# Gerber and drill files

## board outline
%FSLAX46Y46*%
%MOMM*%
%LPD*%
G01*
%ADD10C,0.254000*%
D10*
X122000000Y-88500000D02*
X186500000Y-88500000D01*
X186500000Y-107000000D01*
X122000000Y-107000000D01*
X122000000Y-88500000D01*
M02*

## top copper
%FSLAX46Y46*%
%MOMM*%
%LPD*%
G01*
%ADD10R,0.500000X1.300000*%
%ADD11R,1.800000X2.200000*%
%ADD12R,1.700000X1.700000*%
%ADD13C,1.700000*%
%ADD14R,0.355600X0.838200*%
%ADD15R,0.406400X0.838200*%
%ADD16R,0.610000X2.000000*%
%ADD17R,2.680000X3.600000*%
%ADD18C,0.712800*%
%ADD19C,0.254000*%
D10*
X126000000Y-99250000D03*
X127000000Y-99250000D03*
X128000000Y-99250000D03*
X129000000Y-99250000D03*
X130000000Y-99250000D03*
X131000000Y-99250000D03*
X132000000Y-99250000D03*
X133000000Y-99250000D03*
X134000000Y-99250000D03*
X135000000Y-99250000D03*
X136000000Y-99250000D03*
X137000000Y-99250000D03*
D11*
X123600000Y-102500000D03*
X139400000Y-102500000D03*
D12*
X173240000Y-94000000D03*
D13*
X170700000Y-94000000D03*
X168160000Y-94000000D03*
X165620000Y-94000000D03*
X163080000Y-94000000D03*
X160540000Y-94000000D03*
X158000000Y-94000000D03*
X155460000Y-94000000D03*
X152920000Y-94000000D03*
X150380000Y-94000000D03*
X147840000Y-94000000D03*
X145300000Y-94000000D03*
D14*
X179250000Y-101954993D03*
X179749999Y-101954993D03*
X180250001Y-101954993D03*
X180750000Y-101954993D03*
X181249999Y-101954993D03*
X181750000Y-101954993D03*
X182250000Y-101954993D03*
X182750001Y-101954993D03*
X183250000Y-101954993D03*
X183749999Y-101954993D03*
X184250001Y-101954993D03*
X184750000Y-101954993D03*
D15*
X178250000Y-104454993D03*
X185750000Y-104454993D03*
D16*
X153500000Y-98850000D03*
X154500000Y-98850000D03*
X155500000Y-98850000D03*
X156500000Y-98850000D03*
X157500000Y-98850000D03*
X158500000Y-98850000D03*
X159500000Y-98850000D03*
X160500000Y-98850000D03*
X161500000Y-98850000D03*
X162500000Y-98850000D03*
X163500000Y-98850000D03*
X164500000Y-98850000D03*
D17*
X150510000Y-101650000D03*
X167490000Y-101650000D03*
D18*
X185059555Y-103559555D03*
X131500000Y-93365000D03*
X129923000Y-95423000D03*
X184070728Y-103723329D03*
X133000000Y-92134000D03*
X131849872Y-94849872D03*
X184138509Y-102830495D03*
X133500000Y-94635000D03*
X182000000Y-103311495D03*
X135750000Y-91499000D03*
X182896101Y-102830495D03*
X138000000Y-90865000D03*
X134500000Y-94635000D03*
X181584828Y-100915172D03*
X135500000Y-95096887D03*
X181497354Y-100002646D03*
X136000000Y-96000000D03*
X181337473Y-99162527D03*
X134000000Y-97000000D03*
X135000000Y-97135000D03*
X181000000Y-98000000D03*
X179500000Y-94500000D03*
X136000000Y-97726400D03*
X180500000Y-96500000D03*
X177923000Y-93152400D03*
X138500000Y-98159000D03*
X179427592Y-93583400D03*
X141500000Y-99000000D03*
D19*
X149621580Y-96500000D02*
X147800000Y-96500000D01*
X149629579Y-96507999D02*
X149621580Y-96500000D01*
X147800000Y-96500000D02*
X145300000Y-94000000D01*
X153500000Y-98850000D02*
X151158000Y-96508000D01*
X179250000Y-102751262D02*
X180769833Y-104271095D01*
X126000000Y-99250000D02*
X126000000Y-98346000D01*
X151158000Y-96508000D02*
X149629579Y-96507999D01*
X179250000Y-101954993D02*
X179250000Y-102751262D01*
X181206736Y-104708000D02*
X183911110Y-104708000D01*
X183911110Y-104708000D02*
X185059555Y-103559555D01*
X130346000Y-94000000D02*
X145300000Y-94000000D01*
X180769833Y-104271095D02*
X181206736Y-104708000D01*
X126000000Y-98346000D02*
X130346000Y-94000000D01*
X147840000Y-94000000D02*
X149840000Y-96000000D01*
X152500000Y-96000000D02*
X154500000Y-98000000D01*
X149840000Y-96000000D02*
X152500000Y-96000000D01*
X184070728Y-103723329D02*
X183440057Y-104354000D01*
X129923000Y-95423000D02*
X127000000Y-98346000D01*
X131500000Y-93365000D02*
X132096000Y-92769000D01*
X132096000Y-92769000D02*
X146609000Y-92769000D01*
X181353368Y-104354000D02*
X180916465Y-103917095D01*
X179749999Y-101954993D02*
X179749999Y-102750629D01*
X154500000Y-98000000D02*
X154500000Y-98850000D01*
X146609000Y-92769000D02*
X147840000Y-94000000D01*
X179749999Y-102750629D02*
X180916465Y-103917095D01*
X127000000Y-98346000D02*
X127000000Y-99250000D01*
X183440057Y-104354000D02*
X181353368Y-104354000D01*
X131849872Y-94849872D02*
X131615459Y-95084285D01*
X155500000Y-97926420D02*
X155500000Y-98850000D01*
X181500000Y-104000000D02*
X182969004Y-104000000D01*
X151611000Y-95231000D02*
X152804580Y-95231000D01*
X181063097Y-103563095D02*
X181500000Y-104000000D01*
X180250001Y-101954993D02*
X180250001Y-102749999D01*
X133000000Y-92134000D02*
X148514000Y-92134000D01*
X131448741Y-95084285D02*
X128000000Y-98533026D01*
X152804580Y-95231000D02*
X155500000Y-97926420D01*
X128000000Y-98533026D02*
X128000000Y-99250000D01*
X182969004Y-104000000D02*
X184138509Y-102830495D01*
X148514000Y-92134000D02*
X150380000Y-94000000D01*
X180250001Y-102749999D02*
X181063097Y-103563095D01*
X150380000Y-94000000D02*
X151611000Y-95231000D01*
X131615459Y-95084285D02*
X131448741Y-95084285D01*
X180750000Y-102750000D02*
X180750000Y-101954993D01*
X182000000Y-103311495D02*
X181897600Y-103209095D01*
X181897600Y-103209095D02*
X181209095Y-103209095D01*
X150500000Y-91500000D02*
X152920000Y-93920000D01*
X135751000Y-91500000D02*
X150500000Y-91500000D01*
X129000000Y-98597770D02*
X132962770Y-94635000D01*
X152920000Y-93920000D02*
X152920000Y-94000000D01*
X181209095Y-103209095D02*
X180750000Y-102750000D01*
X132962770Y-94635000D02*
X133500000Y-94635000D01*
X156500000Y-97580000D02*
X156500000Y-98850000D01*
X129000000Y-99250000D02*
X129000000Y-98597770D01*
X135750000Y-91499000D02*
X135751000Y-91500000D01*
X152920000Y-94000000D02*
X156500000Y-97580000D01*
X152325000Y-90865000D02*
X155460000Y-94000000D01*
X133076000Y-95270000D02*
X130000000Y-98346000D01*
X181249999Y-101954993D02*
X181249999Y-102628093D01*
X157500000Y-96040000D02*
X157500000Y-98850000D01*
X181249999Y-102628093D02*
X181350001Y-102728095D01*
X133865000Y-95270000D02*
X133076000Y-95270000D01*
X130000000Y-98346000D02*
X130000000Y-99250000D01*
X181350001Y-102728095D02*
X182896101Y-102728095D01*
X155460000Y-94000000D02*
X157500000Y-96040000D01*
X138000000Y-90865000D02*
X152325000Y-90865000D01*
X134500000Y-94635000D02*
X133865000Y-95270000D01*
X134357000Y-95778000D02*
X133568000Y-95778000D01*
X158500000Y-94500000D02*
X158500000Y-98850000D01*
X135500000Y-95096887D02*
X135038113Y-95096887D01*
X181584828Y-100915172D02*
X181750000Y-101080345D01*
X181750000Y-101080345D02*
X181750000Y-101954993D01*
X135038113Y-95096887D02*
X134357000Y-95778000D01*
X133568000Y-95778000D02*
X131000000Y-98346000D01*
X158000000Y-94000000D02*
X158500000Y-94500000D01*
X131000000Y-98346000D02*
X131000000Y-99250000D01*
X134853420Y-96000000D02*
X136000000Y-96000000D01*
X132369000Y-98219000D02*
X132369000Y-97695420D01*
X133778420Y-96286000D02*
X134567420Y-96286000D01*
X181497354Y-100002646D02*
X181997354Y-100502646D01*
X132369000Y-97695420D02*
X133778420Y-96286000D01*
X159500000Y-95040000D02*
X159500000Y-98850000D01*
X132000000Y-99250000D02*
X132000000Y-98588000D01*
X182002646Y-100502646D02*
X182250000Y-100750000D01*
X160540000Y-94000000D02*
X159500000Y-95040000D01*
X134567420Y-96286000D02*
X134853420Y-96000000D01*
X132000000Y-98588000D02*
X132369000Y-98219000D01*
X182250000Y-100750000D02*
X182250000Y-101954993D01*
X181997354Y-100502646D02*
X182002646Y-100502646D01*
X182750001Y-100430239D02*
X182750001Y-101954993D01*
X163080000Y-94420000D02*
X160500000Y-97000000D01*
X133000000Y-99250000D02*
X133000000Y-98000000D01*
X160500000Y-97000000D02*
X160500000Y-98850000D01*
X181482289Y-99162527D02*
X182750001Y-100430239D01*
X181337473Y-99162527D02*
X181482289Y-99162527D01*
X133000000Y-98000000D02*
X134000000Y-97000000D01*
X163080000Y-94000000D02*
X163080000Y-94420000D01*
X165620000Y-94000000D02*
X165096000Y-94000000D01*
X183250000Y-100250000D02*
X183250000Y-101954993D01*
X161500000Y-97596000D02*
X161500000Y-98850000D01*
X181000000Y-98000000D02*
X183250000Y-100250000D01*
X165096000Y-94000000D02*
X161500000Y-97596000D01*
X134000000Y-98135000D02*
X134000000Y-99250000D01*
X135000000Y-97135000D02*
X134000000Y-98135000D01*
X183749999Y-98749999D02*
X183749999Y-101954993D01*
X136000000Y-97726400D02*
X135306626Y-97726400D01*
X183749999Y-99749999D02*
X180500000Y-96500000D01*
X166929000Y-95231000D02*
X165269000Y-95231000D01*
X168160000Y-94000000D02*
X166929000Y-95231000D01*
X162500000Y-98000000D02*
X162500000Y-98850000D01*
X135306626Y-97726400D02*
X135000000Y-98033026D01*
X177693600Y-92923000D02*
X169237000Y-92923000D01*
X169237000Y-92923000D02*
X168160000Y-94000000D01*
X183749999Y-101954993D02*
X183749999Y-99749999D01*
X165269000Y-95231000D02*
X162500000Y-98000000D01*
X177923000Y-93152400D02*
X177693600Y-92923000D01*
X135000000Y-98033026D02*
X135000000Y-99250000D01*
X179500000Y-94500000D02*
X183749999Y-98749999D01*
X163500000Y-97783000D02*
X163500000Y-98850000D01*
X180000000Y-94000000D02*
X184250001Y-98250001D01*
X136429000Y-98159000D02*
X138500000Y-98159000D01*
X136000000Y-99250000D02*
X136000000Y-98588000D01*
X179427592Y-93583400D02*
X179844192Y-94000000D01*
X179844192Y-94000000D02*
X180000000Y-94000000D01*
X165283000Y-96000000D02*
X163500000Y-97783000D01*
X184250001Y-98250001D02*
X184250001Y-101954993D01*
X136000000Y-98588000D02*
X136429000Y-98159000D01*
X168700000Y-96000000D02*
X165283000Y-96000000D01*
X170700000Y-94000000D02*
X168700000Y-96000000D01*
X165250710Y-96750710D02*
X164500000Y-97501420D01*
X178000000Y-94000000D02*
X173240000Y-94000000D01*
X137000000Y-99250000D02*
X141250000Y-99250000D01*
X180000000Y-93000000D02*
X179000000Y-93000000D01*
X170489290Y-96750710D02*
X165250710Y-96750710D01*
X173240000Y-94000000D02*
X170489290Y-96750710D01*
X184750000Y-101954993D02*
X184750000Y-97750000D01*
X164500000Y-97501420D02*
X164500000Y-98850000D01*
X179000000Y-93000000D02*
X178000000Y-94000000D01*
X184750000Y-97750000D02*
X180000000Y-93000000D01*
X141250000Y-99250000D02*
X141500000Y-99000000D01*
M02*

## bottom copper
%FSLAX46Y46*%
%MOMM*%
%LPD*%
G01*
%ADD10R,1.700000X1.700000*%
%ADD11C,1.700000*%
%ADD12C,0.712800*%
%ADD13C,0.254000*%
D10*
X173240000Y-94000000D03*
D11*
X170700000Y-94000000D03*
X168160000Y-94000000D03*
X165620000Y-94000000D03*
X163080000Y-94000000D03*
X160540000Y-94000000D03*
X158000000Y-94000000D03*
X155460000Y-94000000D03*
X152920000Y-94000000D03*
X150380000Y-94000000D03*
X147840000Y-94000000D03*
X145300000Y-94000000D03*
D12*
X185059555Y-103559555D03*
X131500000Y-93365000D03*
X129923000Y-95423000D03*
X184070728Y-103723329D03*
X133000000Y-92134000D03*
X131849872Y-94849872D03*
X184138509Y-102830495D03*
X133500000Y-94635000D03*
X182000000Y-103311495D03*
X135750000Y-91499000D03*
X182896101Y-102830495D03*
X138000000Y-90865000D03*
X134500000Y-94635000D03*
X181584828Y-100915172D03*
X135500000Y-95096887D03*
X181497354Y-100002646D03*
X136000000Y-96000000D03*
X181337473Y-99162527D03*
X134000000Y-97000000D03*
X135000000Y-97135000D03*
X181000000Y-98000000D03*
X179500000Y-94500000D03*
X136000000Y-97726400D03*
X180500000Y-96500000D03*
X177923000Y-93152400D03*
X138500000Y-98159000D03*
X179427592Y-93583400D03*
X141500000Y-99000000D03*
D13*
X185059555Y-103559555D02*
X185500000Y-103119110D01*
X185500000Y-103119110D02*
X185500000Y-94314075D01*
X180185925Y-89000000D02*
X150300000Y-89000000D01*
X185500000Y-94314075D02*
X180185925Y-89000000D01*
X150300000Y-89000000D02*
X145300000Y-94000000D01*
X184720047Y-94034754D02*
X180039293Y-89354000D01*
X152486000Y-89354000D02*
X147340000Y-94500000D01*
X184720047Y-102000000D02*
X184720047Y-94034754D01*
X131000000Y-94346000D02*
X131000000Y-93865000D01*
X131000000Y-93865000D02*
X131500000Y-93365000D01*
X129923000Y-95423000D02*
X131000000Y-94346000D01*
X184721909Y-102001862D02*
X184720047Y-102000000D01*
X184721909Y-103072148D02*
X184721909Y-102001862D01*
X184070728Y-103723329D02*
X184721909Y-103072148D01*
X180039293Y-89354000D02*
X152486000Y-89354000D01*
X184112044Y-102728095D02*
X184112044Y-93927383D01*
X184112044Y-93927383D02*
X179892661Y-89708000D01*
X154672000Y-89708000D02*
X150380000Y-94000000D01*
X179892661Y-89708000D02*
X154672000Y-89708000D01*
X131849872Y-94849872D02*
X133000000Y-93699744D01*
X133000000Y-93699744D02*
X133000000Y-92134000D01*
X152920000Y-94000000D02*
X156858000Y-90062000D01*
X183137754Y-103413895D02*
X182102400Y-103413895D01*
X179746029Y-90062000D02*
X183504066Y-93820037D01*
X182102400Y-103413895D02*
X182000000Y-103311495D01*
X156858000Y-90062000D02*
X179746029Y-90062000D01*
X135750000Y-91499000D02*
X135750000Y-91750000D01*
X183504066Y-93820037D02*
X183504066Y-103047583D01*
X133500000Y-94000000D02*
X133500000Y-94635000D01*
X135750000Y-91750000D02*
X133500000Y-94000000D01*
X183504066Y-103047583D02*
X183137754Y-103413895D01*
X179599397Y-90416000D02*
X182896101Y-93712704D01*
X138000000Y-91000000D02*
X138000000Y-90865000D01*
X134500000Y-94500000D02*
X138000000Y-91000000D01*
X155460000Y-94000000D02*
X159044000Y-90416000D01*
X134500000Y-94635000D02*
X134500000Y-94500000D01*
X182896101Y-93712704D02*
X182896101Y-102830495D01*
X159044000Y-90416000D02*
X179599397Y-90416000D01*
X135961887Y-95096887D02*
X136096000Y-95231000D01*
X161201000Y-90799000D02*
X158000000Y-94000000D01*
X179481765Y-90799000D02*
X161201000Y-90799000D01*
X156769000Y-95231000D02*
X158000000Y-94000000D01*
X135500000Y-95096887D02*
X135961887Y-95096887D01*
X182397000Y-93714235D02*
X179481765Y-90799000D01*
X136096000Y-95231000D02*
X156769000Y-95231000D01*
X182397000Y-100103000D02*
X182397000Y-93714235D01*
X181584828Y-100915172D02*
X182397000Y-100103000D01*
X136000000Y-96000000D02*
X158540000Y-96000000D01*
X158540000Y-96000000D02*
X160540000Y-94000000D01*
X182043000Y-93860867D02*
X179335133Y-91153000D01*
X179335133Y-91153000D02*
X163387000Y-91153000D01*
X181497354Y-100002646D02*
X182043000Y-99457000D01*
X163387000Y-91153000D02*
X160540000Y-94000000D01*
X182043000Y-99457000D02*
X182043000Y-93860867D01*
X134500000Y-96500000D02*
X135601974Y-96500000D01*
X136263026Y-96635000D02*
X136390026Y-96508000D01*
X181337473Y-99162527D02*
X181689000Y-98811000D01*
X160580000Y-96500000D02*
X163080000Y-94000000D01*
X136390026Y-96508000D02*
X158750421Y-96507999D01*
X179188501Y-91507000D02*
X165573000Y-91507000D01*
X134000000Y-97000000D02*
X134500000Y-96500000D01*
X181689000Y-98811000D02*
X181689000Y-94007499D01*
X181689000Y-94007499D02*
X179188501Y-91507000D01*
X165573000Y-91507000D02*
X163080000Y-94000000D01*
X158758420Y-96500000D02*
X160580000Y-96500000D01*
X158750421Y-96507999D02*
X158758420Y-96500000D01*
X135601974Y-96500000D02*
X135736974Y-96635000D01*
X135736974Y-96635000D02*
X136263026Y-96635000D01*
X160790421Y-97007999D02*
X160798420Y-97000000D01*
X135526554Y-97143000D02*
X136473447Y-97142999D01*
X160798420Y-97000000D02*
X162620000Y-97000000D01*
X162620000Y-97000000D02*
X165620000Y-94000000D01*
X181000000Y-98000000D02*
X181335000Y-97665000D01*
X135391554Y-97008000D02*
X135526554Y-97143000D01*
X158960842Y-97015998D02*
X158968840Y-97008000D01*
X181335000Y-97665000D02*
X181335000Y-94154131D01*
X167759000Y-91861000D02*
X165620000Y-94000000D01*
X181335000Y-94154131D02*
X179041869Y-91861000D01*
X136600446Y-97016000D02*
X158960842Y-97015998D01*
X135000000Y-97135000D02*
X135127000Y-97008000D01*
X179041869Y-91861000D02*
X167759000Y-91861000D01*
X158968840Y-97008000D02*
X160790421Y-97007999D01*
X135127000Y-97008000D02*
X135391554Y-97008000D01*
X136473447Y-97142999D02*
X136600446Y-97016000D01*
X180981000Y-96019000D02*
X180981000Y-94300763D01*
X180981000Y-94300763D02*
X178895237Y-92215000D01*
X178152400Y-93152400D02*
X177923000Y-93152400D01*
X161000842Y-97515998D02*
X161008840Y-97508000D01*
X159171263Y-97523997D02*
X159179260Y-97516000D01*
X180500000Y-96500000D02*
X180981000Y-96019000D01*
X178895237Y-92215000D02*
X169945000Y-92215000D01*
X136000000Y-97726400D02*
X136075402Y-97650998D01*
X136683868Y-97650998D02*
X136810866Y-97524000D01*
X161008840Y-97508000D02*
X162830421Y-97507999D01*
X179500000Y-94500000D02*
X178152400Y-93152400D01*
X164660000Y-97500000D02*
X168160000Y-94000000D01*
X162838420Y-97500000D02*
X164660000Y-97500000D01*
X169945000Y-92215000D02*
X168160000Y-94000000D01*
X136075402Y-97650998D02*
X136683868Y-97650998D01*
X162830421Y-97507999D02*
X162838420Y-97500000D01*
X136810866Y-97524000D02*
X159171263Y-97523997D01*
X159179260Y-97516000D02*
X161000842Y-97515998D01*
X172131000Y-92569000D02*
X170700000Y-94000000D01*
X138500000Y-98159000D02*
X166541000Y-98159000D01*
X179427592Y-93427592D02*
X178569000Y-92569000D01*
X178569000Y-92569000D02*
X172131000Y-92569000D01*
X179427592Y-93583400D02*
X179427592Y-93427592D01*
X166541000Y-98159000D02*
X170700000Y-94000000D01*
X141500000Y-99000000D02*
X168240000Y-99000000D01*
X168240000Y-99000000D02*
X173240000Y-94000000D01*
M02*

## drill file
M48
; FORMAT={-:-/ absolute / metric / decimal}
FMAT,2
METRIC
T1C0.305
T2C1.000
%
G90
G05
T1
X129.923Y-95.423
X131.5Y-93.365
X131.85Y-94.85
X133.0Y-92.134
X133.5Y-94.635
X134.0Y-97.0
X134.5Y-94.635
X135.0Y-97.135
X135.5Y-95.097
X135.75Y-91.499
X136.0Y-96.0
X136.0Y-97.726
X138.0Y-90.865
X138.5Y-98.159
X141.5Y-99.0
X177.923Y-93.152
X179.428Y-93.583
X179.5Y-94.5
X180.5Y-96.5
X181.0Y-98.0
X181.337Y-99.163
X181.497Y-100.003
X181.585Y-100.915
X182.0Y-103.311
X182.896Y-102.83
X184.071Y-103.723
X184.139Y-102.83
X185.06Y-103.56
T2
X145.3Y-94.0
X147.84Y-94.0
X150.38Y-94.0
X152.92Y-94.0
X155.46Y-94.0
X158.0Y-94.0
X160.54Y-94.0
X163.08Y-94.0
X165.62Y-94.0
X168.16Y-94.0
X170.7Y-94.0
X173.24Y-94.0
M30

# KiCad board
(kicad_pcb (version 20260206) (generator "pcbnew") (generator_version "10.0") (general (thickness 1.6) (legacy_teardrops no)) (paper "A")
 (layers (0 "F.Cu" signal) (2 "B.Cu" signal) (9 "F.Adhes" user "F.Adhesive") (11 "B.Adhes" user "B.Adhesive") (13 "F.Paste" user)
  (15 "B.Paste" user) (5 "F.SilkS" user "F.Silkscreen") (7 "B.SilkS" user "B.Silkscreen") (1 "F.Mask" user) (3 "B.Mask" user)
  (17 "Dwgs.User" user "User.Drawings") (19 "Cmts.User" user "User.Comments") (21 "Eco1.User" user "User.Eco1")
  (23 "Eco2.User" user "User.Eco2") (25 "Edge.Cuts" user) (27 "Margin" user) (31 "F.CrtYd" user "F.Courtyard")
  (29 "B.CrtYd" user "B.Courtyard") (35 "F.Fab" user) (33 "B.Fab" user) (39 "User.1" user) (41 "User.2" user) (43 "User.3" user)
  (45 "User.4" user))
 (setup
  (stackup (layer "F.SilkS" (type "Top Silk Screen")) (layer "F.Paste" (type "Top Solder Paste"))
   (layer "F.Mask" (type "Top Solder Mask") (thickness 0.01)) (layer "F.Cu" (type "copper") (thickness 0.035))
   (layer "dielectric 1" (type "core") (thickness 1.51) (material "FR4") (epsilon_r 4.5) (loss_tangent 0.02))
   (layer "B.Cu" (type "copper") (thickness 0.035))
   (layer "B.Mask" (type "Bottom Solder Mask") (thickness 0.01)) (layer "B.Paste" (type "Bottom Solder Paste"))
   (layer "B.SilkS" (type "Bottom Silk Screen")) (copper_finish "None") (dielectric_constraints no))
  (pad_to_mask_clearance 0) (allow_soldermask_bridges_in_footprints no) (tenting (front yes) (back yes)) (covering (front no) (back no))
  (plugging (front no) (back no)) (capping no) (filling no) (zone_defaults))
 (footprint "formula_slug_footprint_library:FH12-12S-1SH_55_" (layer "F.Cu") (at 131.5 100.05)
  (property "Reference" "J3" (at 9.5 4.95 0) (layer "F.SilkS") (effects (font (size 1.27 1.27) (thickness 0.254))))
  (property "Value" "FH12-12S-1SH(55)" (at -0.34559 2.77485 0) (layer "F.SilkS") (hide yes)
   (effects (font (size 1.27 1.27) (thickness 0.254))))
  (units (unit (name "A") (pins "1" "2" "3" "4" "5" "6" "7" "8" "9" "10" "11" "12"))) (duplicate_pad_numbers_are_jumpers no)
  (pad "1" smd rect (at -5.5 -0.8) (size 0.5 1.3) (layers "F.Cu" "F.Mask" "F.Paste") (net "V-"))
  (pad "2" smd rect (at -4.5 -0.8) (size 0.5 1.3) (layers "F.Cu" "F.Mask" "F.Paste") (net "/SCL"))
  (pad "3" smd rect (at -3.5 -0.8) (size 0.5 1.3) (layers "F.Cu" "F.Mask" "F.Paste") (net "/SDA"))
  (pad "4" smd rect (at -2.5 -0.8) (size 0.5 1.3) (layers "F.Cu" "F.Mask" "F.Paste") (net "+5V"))
  (pad "5" smd rect (at -1.5 -0.8) (size 0.5 1.3) (layers "F.Cu" "F.Mask" "F.Paste") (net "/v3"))
  (pad "6" smd rect (at -0.5 -0.8) (size 0.5 1.3) (layers "F.Cu" "F.Mask" "F.Paste") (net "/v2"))
  (pad "7" smd rect (at 0.5 -0.8) (size 0.5 1.3) (layers "F.Cu" "F.Mask" "F.Paste") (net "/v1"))
  (pad "8" smd rect (at 1.5 -0.8) (size 0.5 1.3) (layers "F.Cu" "F.Mask" "F.Paste") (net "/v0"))
  (pad "9" smd rect (at 2.5 -0.8) (size 0.5 1.3) (layers "F.Cu" "F.Mask" "F.Paste") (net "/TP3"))
  (pad "10" smd rect (at 3.5 -0.8) (size 0.5 1.3) (layers "F.Cu" "F.Mask" "F.Paste") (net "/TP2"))
  (pad "11" smd rect (at 4.5 -0.8) (size 0.5 1.3) (layers "F.Cu" "F.Mask" "F.Paste") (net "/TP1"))
  (pad "12" smd rect (at 5.5 -0.8) (size 0.5 1.3) (layers "F.Cu" "F.Mask" "F.Paste") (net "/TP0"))
  (pad "13" smd rect (at -7.9 2.45) (size 1.8 2.2) (layers "F.Cu" "F.Mask" "F.Paste"))
  (pad "14" smd rect (at 7.9 2.45) (size 1.8 2.2) (layers "F.Cu" "F.Mask" "F.Paste")))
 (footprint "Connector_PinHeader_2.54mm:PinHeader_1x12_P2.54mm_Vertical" (layer "F.Cu") (at 173.24 94 -90)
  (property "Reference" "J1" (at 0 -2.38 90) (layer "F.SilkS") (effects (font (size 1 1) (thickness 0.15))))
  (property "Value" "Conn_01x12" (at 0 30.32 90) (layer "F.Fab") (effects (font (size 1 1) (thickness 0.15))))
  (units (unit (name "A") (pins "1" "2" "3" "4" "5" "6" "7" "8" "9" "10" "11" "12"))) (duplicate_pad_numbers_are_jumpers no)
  (pad "1" thru_hole rect (at 0 0 270) (size 1.7 1.7) (drill 1) (layers "*.Cu" "*.Mask") (remove_unused_layers no) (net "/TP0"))
  (pad "2" thru_hole circle (at 0 2.54 270) (size 1.7 1.7) (drill 1) (layers "*.Cu" "*.Mask") (remove_unused_layers no) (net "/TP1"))
  (pad "3" thru_hole circle (at 0 5.08 270) (size 1.7 1.7) (drill 1) (layers "*.Cu" "*.Mask") (remove_unused_layers no) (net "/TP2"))
  (pad "4" thru_hole circle (at 0 7.62 270) (size 1.7 1.7) (drill 1) (layers "*.Cu" "*.Mask") (remove_unused_layers no) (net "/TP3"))
  (pad "5" thru_hole circle (at 0 10.16 270) (size 1.7 1.7) (drill 1) (layers "*.Cu" "*.Mask") (remove_unused_layers no) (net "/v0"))
  (pad "6" thru_hole circle (at 0 12.7 270) (size 1.7 1.7) (drill 1) (layers "*.Cu" "*.Mask") (remove_unused_layers no) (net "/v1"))
  (pad "7" thru_hole circle (at 0 15.24 270) (size 1.7 1.7) (drill 1) (layers "*.Cu" "*.Mask") (remove_unused_layers no) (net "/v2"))
  (pad "8" thru_hole circle (at 0 17.78 270) (size 1.7 1.7) (drill 1) (layers "*.Cu" "*.Mask") (remove_unused_layers no) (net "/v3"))
  (pad "9" thru_hole circle (at 0 20.32 270) (size 1.7 1.7) (drill 1) (layers "*.Cu" "*.Mask") (remove_unused_layers no) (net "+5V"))
  (pad "10" thru_hole circle (at 0 22.86 270) (size 1.7 1.7) (drill 1) (layers "*.Cu" "*.Mask") (remove_unused_layers no) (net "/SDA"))
  (pad "11" thru_hole circle (at 0 25.4 270) (size 1.7 1.7) (drill 1) (layers "*.Cu" "*.Mask") (remove_unused_layers no) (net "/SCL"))
  (pad "12" thru_hole circle (at 0 27.94 270) (size 1.7 1.7) (drill 1) (layers "*.Cu" "*.Mask") (remove_unused_layers no) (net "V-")))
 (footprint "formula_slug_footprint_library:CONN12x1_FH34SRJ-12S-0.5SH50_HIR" (layer "F.Cu") (at 182 103)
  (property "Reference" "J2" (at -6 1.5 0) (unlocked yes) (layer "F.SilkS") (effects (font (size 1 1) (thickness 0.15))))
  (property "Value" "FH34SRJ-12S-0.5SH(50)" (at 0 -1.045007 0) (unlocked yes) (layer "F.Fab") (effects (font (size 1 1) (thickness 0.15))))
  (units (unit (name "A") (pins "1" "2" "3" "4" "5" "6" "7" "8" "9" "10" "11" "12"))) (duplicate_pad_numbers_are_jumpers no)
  (pad "1" smd rect (at -2.75 -1.045007) (size 0.3556 0.8382) (layers "F.Cu" "F.Mask" "F.Paste") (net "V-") (clearance 0.1))
  (pad "2" smd rect (at -2.250001 -1.045007) (size 0.3556 0.8382) (layers "F.Cu" "F.Mask" "F.Paste") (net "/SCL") (clearance 0.1))
  (pad "3" smd rect (at -1.749999 -1.045007) (size 0.3556 0.8382) (layers "F.Cu" "F.Mask" "F.Paste") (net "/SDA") (clearance 0.1))
  (pad "4" smd rect (at -1.25 -1.045007) (size 0.3556 0.8382) (layers "F.Cu" "F.Mask" "F.Paste") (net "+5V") (clearance 0.1))
  (pad "5" smd rect (at -0.750001 -1.045007) (size 0.3556 0.8382) (layers "F.Cu" "F.Mask" "F.Paste") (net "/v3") (clearance 0.1))
  (pad "6" smd rect (at -0.25 -1.045007) (size 0.3556 0.8382) (layers "F.Cu" "F.Mask" "F.Paste") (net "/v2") (clearance 0.1))
  (pad "7" smd rect (at 0.25 -1.045007) (size 0.3556 0.8382) (layers "F.Cu" "F.Mask" "F.Paste") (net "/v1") (clearance 0.1))
  (pad "8" smd rect (at 0.750001 -1.045007) (size 0.3556 0.8382) (layers "F.Cu" "F.Mask" "F.Paste") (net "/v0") (clearance 0.1))
  (pad "9" smd rect (at 1.25 -1.045007) (size 0.3556 0.8382) (layers "F.Cu" "F.Mask" "F.Paste") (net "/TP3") (clearance 0.1))
  (pad "10" smd rect (at 1.749999 -1.045007) (size 0.3556 0.8382) (layers "F.Cu" "F.Mask" "F.Paste") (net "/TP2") (clearance 0.1))
  (pad "11" smd rect (at 2.250001 -1.045007) (size 0.3556 0.8382) (layers "F.Cu" "F.Mask" "F.Paste") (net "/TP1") (clearance 0.1))
  (pad "12" smd rect (at 2.75 -1.045007) (size 0.3556 0.8382) (layers "F.Cu" "F.Mask" "F.Paste") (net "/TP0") (clearance 0.1))
  (pad "13" smd rect (at -3.75 1.454993) (size 0.4064 0.8382) (layers "F.Cu" "F.Mask" "F.Paste"))
  (pad "14" smd rect (at 3.75 1.454993) (size 0.4064 0.8382) (layers "F.Cu" "F.Mask" "F.Paste")))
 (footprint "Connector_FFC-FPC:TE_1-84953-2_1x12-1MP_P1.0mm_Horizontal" (layer "F.Cu") (at 159 100.65)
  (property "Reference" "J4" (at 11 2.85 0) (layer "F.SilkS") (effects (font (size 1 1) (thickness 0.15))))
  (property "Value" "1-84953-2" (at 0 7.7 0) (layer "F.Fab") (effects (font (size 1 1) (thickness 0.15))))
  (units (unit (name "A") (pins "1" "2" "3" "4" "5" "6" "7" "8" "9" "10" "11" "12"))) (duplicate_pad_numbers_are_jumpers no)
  (pad "1" smd rect (at -5.5 -1.8) (size 0.61 2) (layers "F.Cu" "F.Mask" "F.Paste") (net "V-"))
  (pad "2" smd rect (at -4.5 -1.8) (size 0.61 2) (layers "F.Cu" "F.Mask" "F.Paste") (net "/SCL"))
  (pad "3" smd rect (at -3.5 -1.8) (size 0.61 2) (layers "F.Cu" "F.Mask" "F.Paste") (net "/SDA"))
  (pad "4" smd rect (at -2.5 -1.8) (size 0.61 2) (layers "F.Cu" "F.Mask" "F.Paste") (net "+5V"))
  (pad "5" smd rect (at -1.5 -1.8) (size 0.61 2) (layers "F.Cu" "F.Mask" "F.Paste") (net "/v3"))
  (pad "6" smd rect (at -0.5 -1.8) (size 0.61 2) (layers "F.Cu" "F.Mask" "F.Paste") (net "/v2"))
  (pad "7" smd rect (at 0.5 -1.8) (size 0.61 2) (layers "F.Cu" "F.Mask" "F.Paste") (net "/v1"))
  (pad "8" smd rect (at 1.5 -1.8) (size 0.61 2) (layers "F.Cu" "F.Mask" "F.Paste") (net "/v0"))
  (pad "9" smd rect (at 2.5 -1.8) (size 0.61 2) (layers "F.Cu" "F.Mask" "F.Paste") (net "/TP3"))
  (pad "10" smd rect (at 3.5 -1.8) (size 0.61 2) (layers "F.Cu" "F.Mask" "F.Paste") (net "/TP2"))
  (pad "11" smd rect (at 4.5 -1.8) (size 0.61 2) (layers "F.Cu" "F.Mask" "F.Paste") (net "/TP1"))
  (pad "12" smd rect (at 5.5 -1.8) (size 0.61 2) (layers "F.Cu" "F.Mask" "F.Paste") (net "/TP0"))
  (pad "MP" smd rect (at -8.49 1) (size 2.68 3.6) (layers "F.Cu" "F.Mask" "F.Paste"))
  (pad "MP" smd rect (at 8.49 1) (size 2.68 3.6) (layers "F.Cu" "F.Mask" "F.Paste")))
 (gr_rect (start 122 88.5) (end 186.5 107) (stroke (width 0.254) (type solid)) (fill no) (layer "Edge.Cuts"))
 (segment (start 149.62158 96.5) (end 147.8 96.5) (width 0.254) (layer "F.Cu") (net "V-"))
 (segment (start 149.629579 96.507999) (end 149.62158 96.5) (width 0.254) (layer "F.Cu") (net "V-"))
 (segment (start 147.8 96.5) (end 145.3 94) (width 0.254) (layer "F.Cu") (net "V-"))
 (segment (start 153.5 98.85) (end 151.158 96.508) (width 0.254) (layer "F.Cu") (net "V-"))
 (segment (start 179.25 102.751262) (end 180.769833 104.271095) (width 0.254) (layer "F.Cu") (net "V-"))
 (segment (start 126 99.25) (end 126 98.346) (width 0.254) (layer "F.Cu") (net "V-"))
 (segment (start 151.158 96.508) (end 149.629579 96.507999) (width 0.254) (layer "F.Cu") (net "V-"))
 (segment (start 179.25 101.954993) (end 179.25 102.751262) (width 0.254) (layer "F.Cu") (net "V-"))
 (segment (start 181.206736 104.708) (end 183.91111 104.708) (width 0.254) (layer "F.Cu") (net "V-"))
 (segment (start 183.91111 104.708) (end 185.059555 103.559555) (width 0.254) (layer "F.Cu") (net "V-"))
 (segment (start 130.346 94) (end 145.3 94) (width 0.254) (layer "F.Cu") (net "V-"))
 (segment (start 180.769833 104.271095) (end 181.206736 104.708) (width 0.254) (layer "F.Cu") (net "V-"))
 (segment (start 126 98.346) (end 130.346 94) (width 0.254) (layer "F.Cu") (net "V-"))
 (via (at 185.059555 103.559555) (size 0.7128) (drill 0.3048) (layers "F.Cu" "B.Cu") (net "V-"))
 (segment (start 185.059555 103.559555) (end 185.5 103.11911) (width 0.254) (layer "B.Cu") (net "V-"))
 (segment (start 185.5 103.11911) (end 185.5 94.314075) (width 0.254) (layer "B.Cu") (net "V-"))
 (segment (start 180.185925 89) (end 150.3 89) (width 0.254) (layer "B.Cu") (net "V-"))
 (segment (start 185.5 94.314075) (end 180.185925 89) (width 0.254) (layer "B.Cu") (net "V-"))
 (segment (start 150.3 89) (end 145.3 94) (width 0.254) (layer "B.Cu") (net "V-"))
 (segment (start 147.84 94) (end 149.84 96) (width 0.254) (layer "F.Cu") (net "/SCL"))
 (segment (start 152.5 96) (end 154.5 98) (width 0.254) (layer "F.Cu") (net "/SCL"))
 (segment (start 149.84 96) (end 152.5 96) (width 0.254) (layer "F.Cu") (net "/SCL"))
 (segment (start 184.070728 103.723329) (end 183.440057 104.354) (width 0.254) (layer "F.Cu") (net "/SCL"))
 (segment (start 129.923 95.423) (end 127 98.346) (width 0.254) (layer "F.Cu") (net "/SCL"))
 (segment (start 131.5 93.365) (end 132.096 92.769) (width 0.254) (layer "F.Cu") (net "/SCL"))
 (segment (start 132.096 92.769) (end 146.609 92.769) (width 0.254) (layer "F.Cu") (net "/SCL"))
 (segment (start 181.353368 104.354) (end 180.916465 103.917095) (width 0.254) (layer "F.Cu") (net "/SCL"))
 (segment (start 179.749999 101.954993) (end 179.749999 102.750629) (width 0.254) (layer "F.Cu") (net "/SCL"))
 (segment (start 154.5 98) (end 154.5 98.85) (width 0.254) (layer "F.Cu") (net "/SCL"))
 (segment (start 146.609 92.769) (end 147.84 94) (width 0.254) (layer "F.Cu") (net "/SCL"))
 (segment (start 179.749999 102.750629) (end 180.916465 103.917095) (width 0.254) (layer "F.Cu") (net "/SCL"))
 (segment (start 127 98.346) (end 127 99.25) (width 0.254) (layer "F.Cu") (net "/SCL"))
 (segment (start 183.440057 104.354) (end 181.353368 104.354) (width 0.254) (layer "F.Cu") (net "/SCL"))
 (via (at 131.5 93.365) (size 0.7128) (drill 0.3048) (layers "F.Cu" "B.Cu") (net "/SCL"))
 (via (at 129.923 95.423) (size 0.7128) (drill 0.3048) (layers "F.Cu" "B.Cu") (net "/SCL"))
 (via (at 184.070728 103.723329) (size 0.7128) (drill 0.3048) (layers "F.Cu" "B.Cu") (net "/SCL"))
 (segment (start 184.720047 94.034754) (end 180.039293 89.354) (width 0.254) (layer "B.Cu") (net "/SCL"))
 (segment (start 152.486 89.354) (end 147.34 94.5) (width 0.254) (layer "B.Cu") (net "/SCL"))
 (segment (start 184.720047 102) (end 184.720047 94.034754) (width 0.254) (layer "B.Cu") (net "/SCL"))
 (segment (start 131 94.346) (end 131 93.865) (width 0.254) (layer "B.Cu") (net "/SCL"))
 (segment (start 131 93.865) (end 131.5 93.365) (width 0.254) (layer "B.Cu") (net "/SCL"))
 (segment (start 129.923 95.423) (end 131 94.346) (width 0.254) (layer "B.Cu") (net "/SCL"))
 (segment (start 184.721909 102.001862) (end 184.720047 102) (width 0.254) (layer "B.Cu") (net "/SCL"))
 (segment (start 184.721909 103.072148) (end 184.721909 102.001862) (width 0.254) (layer "B.Cu") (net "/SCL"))
 (segment (start 184.070728 103.723329) (end 184.721909 103.072148) (width 0.254) (layer "B.Cu") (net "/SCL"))
 (segment (start 180.039293 89.354) (end 152.486 89.354) (width 0.254) (layer "B.Cu") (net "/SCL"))
 (segment (start 131.849872 94.849872) (end 131.615459 95.084285) (width 0.254) (layer "F.Cu") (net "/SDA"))
 (segment (start 155.5 97.92642) (end 155.5 98.85) (width 0.254) (layer "F.Cu") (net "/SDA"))
 (segment (start 181.5 104) (end 182.969004 104) (width 0.254) (layer "F.Cu") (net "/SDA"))
 (segment (start 151.611 95.231) (end 152.80458 95.231) (width 0.254) (layer "F.Cu") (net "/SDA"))
 (segment (start 181.063097 103.563095) (end 181.5 104) (width 0.254) (layer "F.Cu") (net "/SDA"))
 (segment (start 180.250001 101.954993) (end 180.250001 102.749999) (width 0.254) (layer "F.Cu") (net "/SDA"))
 (segment (start 133 92.134) (end 148.514 92.134) (width 0.254) (layer "F.Cu") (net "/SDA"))
 (segment (start 131.448741 95.084285) (end 128 98.533026) (width 0.254) (layer "F.Cu") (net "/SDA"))
 (segment (start 152.80458 95.231) (end 155.5 97.92642) (width 0.254) (layer "F.Cu") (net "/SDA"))
 (segment (start 128 98.533026) (end 128 99.25) (width 0.254) (layer "F.Cu") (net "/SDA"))
 (segment (start 182.969004 104) (end 184.138509 102.830495) (width 0.254) (layer "F.Cu") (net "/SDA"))
 (segment (start 148.514 92.134) (end 150.38 94) (width 0.254) (layer "F.Cu") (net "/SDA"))
 (segment (start 180.250001 102.749999) (end 181.063097 103.563095) (width 0.254) (layer "F.Cu") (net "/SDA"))
 (segment (start 150.38 94) (end 151.611 95.231) (width 0.254) (layer "F.Cu") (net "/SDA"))
 (segment (start 131.615459 95.084285) (end 131.448741 95.084285) (width 0.254) (layer "F.Cu") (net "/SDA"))
 (via (at 133 92.134) (size 0.7128) (drill 0.3048) (layers "F.Cu" "B.Cu") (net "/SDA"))
 (via (at 131.849872 94.849872) (size 0.7128) (drill 0.3048) (layers "F.Cu" "B.Cu") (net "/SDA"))
 (via (at 184.138509 102.830495) (size 0.7128) (drill 0.3048) (layers "F.Cu" "B.Cu") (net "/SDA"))
 (segment (start 184.112044 102.728095) (end 184.112044 93.927383) (width 0.254) (layer "B.Cu") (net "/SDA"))
 (segment (start 184.112044 93.927383) (end 179.892661 89.708) (width 0.254) (layer "B.Cu") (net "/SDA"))
 (segment (start 154.672 89.708) (end 150.38 94) (width 0.254) (layer "B.Cu") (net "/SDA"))
 (segment (start 179.892661 89.708) (end 154.672 89.708) (width 0.254) (layer "B.Cu") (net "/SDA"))
 (segment (start 131.849872 94.849872) (end 133 93.699744) (width 0.254) (layer "B.Cu") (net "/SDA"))
 (segment (start 133 93.699744) (end 133 92.134) (width 0.254) (layer "B.Cu") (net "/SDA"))
 (segment (start 180.75 102.75) (end 180.75 101.954993) (width 0.254) (layer "F.Cu") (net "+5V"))
 (segment (start 182 103.311495) (end 181.8976 103.209095) (width 0.254) (layer "F.Cu") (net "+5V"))
 (segment (start 181.8976 103.209095) (end 181.209095 103.209095) (width 0.254) (layer "F.Cu") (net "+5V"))
 (segment (start 150.5 91.5) (end 152.92 93.92) (width 0.254) (layer "F.Cu") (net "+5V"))
 (segment (start 135.751 91.5) (end 150.5 91.5) (width 0.254) (layer "F.Cu") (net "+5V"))
 (segment (start 129 98.59777) (end 132.96277 94.635) (width 0.254) (layer "F.Cu") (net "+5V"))
 (segment (start 152.92 93.92) (end 152.92 94) (width 0.254) (layer "F.Cu") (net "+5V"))
 (segment (start 181.209095 103.209095) (end 180.75 102.75) (width 0.254) (layer "F.Cu") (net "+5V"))
 (segment (start 132.96277 94.635) (end 133.5 94.635) (width 0.254) (layer "F.Cu") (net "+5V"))
 (segment (start 156.5 97.58) (end 156.5 98.85) (width 0.254) (layer "F.Cu") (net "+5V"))
 (segment (start 129 99.25) (end 129 98.59777) (width 0.254) (layer "F.Cu") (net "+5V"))
 (segment (start 135.75 91.499) (end 135.751 91.5) (width 0.254) (layer "F.Cu") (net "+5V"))
 (segment (start 152.92 94) (end 156.5 97.58) (width 0.254) (layer "F.Cu") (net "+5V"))
 (via (at 133.5 94.635) (size 0.7128) (drill 0.3048) (layers "F.Cu" "B.Cu") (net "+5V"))
 (via (at 182 103.311495) (size 0.7128) (drill 0.3048) (layers "F.Cu" "B.Cu") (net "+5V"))
 (via (at 135.75 91.499) (size 0.7128) (drill 0.3048) (layers "F.Cu" "B.Cu") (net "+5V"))
 (segment (start 152.92 94) (end 156.858 90.062) (width 0.254) (layer "B.Cu") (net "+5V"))
 (segment (start 183.137754 103.413895) (end 182.1024 103.413895) (width 0.254) (layer "B.Cu") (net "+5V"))
 (segment (start 179.746029 90.062) (end 183.504066 93.820037) (width 0.254) (layer "B.Cu") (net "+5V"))
 (segment (start 182.1024 103.413895) (end 182 103.311495) (width 0.254) (layer "B.Cu") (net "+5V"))
 (segment (start 156.858 90.062) (end 179.746029 90.062) (width 0.254) (layer "B.Cu") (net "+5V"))
 (segment (start 135.75 91.499) (end 135.75 91.75) (width 0.254) (layer "B.Cu") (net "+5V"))
 (segment (start 183.504066 93.820037) (end 183.504066 103.047583) (width 0.254) (layer "B.Cu") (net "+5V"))
 (segment (start 133.5 94) (end 133.5 94.635) (width 0.254) (layer "B.Cu") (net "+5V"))
 (segment (start 135.75 91.75) (end 133.5 94) (width 0.254) (layer "B.Cu") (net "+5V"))
 (segment (start 183.504066 103.047583) (end 183.137754 103.413895) (width 0.254) (layer "B.Cu") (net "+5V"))
 (segment (start 152.325 90.865) (end 155.46 94) (width 0.254) (layer "F.Cu") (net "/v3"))
 (segment (start 133.076 95.27) (end 130 98.346) (width 0.254) (layer "F.Cu") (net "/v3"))
 (segment (start 181.249999 101.954993) (end 181.249999 102.628093) (width 0.254) (layer "F.Cu") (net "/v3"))
 (segment (start 157.5 96.04) (end 157.5 98.85) (width 0.254) (layer "F.Cu") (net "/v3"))
 (segment (start 181.249999 102.628093) (end 181.350001 102.728095) (width 0.254) (layer "F.Cu") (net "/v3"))
 (segment (start 133.865 95.27) (end 133.076 95.27) (width 0.254) (layer "F.Cu") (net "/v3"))
 (segment (start 130 98.346) (end 130 99.25) (width 0.254) (layer "F.Cu") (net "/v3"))
 (segment (start 181.350001 102.728095) (end 182.896101 102.728095) (width 0.254) (layer "F.Cu") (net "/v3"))
 (segment (start 155.46 94) (end 157.5 96.04) (width 0.254) (layer "F.Cu") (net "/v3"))
 (segment (start 138 90.865) (end 152.325 90.865) (width 0.254) (layer "F.Cu") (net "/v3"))
 (segment (start 134.5 94.635) (end 133.865 95.27) (width 0.254) (layer "F.Cu") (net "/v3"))
 (via (at 182.896101 102.830495) (size 0.7128) (drill 0.3048) (layers "F.Cu" "B.Cu") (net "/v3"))
 (via (at 138 90.865) (size 0.7128) (drill 0.3048) (layers "F.Cu" "B.Cu") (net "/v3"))
 (via (at 134.5 94.635) (size 0.7128) (drill 0.3048) (layers "F.Cu" "B.Cu") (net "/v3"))
 (segment (start 179.599397 90.416) (end 182.896101 93.712704) (width 0.254) (layer "B.Cu") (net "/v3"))
 (segment (start 138 91) (end 138 90.865) (width 0.254) (layer "B.Cu") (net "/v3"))
 (segment (start 134.5 94.5) (end 138 91) (width 0.254) (layer "B.Cu") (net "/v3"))
 (segment (start 155.46 94) (end 159.044 90.416) (width 0.254) (layer "B.Cu") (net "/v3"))
 (segment (start 134.5 94.635) (end 134.5 94.5) (width 0.254) (layer "B.Cu") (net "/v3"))
 (segment (start 182.896101 93.712704) (end 182.896101 102.830495) (width 0.254) (layer "B.Cu") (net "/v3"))
 (segment (start 159.044 90.416) (end 179.599397 90.416) (width 0.254) (layer "B.Cu") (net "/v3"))
 (segment (start 134.357 95.778) (end 133.568 95.778) (width 0.254) (layer "F.Cu") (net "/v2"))
 (segment (start 158.5 94.5) (end 158.5 98.85) (width 0.254) (layer "F.Cu") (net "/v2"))
 (segment (start 135.5 95.096887) (end 135.038113 95.096887) (width 0.254) (layer "F.Cu") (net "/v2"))
 (segment (start 181.584828 100.915172) (end 181.75 101.080345) (width 0.254) (layer "F.Cu") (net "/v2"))
 (segment (start 181.75 101.080345) (end 181.75 101.954993) (width 0.254) (layer "F.Cu") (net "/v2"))
 (segment (start 135.038113 95.096887) (end 134.357 95.778) (width 0.254) (layer "F.Cu") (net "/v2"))
 (segment (start 133.568 95.778) (end 131 98.346) (width 0.254) (layer "F.Cu") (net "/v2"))
 (segment (start 158 94) (end 158.5 94.5) (width 0.254) (layer "F.Cu") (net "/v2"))
 (segment (start 131 98.346) (end 131 99.25) (width 0.254) (layer "F.Cu") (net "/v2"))
 (via (at 181.584828 100.915172) (size 0.7128) (drill 0.3048) (layers "F.Cu" "B.Cu") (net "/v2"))
 (via (at 135.5 95.096887) (size 0.7128) (drill 0.3048) (layers "F.Cu" "B.Cu") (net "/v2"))
 (segment (start 135.961887 95.096887) (end 136.096 95.231) (width 0.254) (layer "B.Cu") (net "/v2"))
 (segment (start 161.201 90.799) (end 158 94) (width 0.254) (layer "B.Cu") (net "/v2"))
 (segment (start 179.481765 90.799) (end 161.201 90.799) (width 0.254) (layer "B.Cu") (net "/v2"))
 (segment (start 156.769 95.231) (end 158 94) (width 0.254) (layer "B.Cu") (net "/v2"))
 (segment (start 135.5 95.096887) (end 135.961887 95.096887) (width 0.254) (layer "B.Cu") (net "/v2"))
 (segment (start 182.397 93.714235) (end 179.481765 90.799) (width 0.254) (layer "B.Cu") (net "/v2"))
 (segment (start 136.096 95.231) (end 156.769 95.231) (width 0.254) (layer "B.Cu") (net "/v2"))
 (segment (start 182.397 100.103) (end 182.397 93.714235) (width 0.254) (layer "B.Cu") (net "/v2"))
 (segment (start 181.584828 100.915172) (end 182.397 100.103) (width 0.254) (layer "B.Cu") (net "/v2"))
 (segment (start 134.85342 96) (end 136 96) (width 0.254) (layer "F.Cu") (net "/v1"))
 (segment (start 132.369 98.219) (end 132.369 97.69542) (width 0.254) (layer "F.Cu") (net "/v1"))
 (segment (start 133.77842 96.286) (end 134.56742 96.286) (width 0.254) (layer "F.Cu") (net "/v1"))
 (segment (start 181.497354 100.002646) (end 181.997354 100.502646) (width 0.254) (layer "F.Cu") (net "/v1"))
 (segment (start 132.369 97.69542) (end 133.77842 96.286) (width 0.254) (layer "F.Cu") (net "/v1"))
 (segment (start 159.5 95.04) (end 159.5 98.85) (width 0.254) (layer "F.Cu") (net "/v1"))
 (segment (start 132 99.25) (end 132 98.588) (width 0.254) (layer "F.Cu") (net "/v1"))
 (segment (start 182.002646 100.502646) (end 182.25 100.75) (width 0.254) (layer "F.Cu") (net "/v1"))
 (segment (start 160.54 94) (end 159.5 95.04) (width 0.254) (layer "F.Cu") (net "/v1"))
 (segment (start 134.56742 96.286) (end 134.85342 96) (width 0.254) (layer "F.Cu") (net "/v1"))
 (segment (start 132 98.588) (end 132.369 98.219) (width 0.254) (layer "F.Cu") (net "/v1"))
 (segment (start 182.25 100.75) (end 182.25 101.954993) (width 0.254) (layer "F.Cu") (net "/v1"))
 (segment (start 181.997354 100.502646) (end 182.002646 100.502646) (width 0.254) (layer "F.Cu") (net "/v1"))
 (via (at 181.497354 100.002646) (size 0.7128) (drill 0.3048) (layers "F.Cu" "B.Cu") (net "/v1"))
 (via (at 136 96) (size 0.7128) (drill 0.3048) (layers "F.Cu" "B.Cu") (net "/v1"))
 (segment (start 136 96) (end 158.54 96) (width 0.254) (layer "B.Cu") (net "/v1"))
 (segment (start 158.54 96) (end 160.54 94) (width 0.254) (layer "B.Cu") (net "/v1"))
 (segment (start 182.043 93.860867) (end 179.335133 91.153) (width 0.254) (layer "B.Cu") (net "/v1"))
 (segment (start 179.335133 91.153) (end 163.387 91.153) (width 0.254) (layer "B.Cu") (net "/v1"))
 (segment (start 181.497354 100.002646) (end 182.043 99.457) (width 0.254) (layer "B.Cu") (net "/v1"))
 (segment (start 163.387 91.153) (end 160.54 94) (width 0.254) (layer "B.Cu") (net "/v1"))
 (segment (start 182.043 99.457) (end 182.043 93.860867) (width 0.254) (layer "B.Cu") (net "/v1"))
 (segment (start 182.750001 100.430239) (end 182.750001 101.954993) (width 0.254) (layer "F.Cu") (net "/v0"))
 (segment (start 163.08 94.42) (end 160.5 97) (width 0.254) (layer "F.Cu") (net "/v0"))
 (segment (start 133 99.25) (end 133 98) (width 0.254) (layer "F.Cu") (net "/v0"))
 (segment (start 160.5 97) (end 160.5 98.85) (width 0.254) (layer "F.Cu") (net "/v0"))
 (segment (start 181.482289 99.162527) (end 182.750001 100.430239) (width 0.254) (layer "F.Cu") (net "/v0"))
 (segment (start 181.337473 99.162527) (end 181.482289 99.162527) (width 0.254) (layer "F.Cu") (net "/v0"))
 (segment (start 133 98) (end 134 97) (width 0.254) (layer "F.Cu") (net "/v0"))
 (segment (start 163.08 94) (end 163.08 94.42) (width 0.254) (layer "F.Cu") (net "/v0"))
 (via (at 181.337473 99.162527) (size 0.7128) (drill 0.3048) (layers "F.Cu" "B.Cu") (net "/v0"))
 (via (at 134 97) (size 0.7128) (drill 0.3048) (layers "F.Cu" "B.Cu") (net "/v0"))
 (segment (start 134.5 96.5) (end 135.601974 96.5) (width 0.254) (layer "B.Cu") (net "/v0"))
 (segment (start 136.263026 96.635) (end 136.390026 96.508) (width 0.254) (layer "B.Cu") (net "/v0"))
 (segment (start 181.337473 99.162527) (end 181.689 98.811) (width 0.254) (layer "B.Cu") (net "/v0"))
 (segment (start 160.58 96.5) (end 163.08 94) (width 0.254) (layer "B.Cu") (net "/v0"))
 (segment (start 136.390026 96.508) (end 158.750421 96.507999) (width 0.254) (layer "B.Cu") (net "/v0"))
 (segment (start 179.188501 91.507) (end 165.573 91.507) (width 0.254) (layer "B.Cu") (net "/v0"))
 (segment (start 134 97) (end 134.5 96.5) (width 0.254) (layer "B.Cu") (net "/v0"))
 (segment (start 181.689 98.811) (end 181.689 94.007499) (width 0.254) (layer "B.Cu") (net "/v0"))
 (segment (start 181.689 94.007499) (end 179.188501 91.507) (width 0.254) (layer "B.Cu") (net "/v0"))
 (segment (start 165.573 91.507) (end 163.08 94) (width 0.254) (layer "B.Cu") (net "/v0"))
 (segment (start 158.75842 96.5) (end 160.58 96.5) (width 0.254) (layer "B.Cu") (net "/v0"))
 (segment (start 158.750421 96.507999) (end 158.75842 96.5) (width 0.254) (layer "B.Cu") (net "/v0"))
 (segment (start 135.601974 96.5) (end 135.736974 96.635) (width 0.254) (layer "B.Cu") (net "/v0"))
 (segment (start 135.736974 96.635) (end 136.263026 96.635) (width 0.254) (layer "B.Cu") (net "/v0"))
 (segment (start 165.62 94) (end 165.096 94) (width 0.254) (layer "F.Cu") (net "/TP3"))
 (segment (start 183.25 100.25) (end 183.25 101.954993) (width 0.254) (layer "F.Cu") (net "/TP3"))
 (segment (start 161.5 97.596) (end 161.5 98.85) (width 0.254) (layer "F.Cu") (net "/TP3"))
 (segment (start 181 98) (end 183.25 100.25) (width 0.254) (layer "F.Cu") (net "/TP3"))
 (segment (start 165.096 94) (end 161.5 97.596) (width 0.254) (layer "F.Cu") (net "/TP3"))
 (segment (start 134 98.135) (end 134 99.25) (width 0.254) (layer "F.Cu") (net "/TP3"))
 (segment (start 135 97.135) (end 134 98.135) (width 0.254) (layer "F.Cu") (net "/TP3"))
 (via (at 135 97.135) (size 0.7128) (drill 0.3048) (layers "F.Cu" "B.Cu") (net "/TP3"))
 (via (at 181 98) (size 0.7128) (drill 0.3048) (layers "F.Cu" "B.Cu") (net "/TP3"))
 (segment (start 160.790421 97.007999) (end 160.79842 97) (width 0.254) (layer "B.Cu") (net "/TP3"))
 (segment (start 135.526554 97.143) (end 136.473447 97.142999) (width 0.254) (layer "B.Cu") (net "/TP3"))
 (segment (start 160.79842 97) (end 162.62 97) (width 0.254) (layer "B.Cu") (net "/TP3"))
 (segment (start 162.62 97) (end 165.62 94) (width 0.254) (layer "B.Cu") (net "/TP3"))
 (segment (start 181 98) (end 181.335 97.665) (width 0.254) (layer "B.Cu") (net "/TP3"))
 (segment (start 135.391554 97.008) (end 135.526554 97.143) (width 0.254) (layer "B.Cu") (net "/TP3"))
 (segment (start 158.960842 97.015998) (end 158.96884 97.008) (width 0.254) (layer "B.Cu") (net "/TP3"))
 (segment (start 181.335 97.665) (end 181.335 94.154131) (width 0.254) (layer "B.Cu") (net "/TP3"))
 (segment (start 167.759 91.861) (end 165.62 94) (width 0.254) (layer "B.Cu") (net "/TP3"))
 (segment (start 181.335 94.154131) (end 179.041869 91.861) (width 0.254) (layer "B.Cu") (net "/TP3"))
 (segment (start 136.600446 97.016) (end 158.960842 97.015998) (width 0.254) (layer "B.Cu") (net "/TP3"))
 (segment (start 135 97.135) (end 135.127 97.008) (width 0.254) (layer "B.Cu") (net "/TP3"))
 (segment (start 179.041869 91.861) (end 167.759 91.861) (width 0.254) (layer "B.Cu") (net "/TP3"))
 (segment (start 158.96884 97.008) (end 160.790421 97.007999) (width 0.254) (layer "B.Cu") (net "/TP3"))
 (segment (start 135.127 97.008) (end 135.391554 97.008) (width 0.254) (layer "B.Cu") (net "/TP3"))
 (segment (start 136.473447 97.142999) (end 136.600446 97.016) (width 0.254) (layer "B.Cu") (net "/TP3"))
 (segment (start 183.749999 98.749999) (end 183.749999 101.954993) (width 0.254) (layer "F.Cu") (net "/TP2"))
 (segment (start 136 97.7264) (end 135.306626 97.7264) (width 0.254) (layer "F.Cu") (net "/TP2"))
 (segment (start 183.749999 99.749999) (end 180.5 96.5) (width 0.254) (layer "F.Cu") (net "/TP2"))
 (segment (start 166.929 95.231) (end 165.269 95.231) (width 0.254) (layer "F.Cu") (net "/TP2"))
 (segment (start 168.16 94) (end 166.929 95.231) (width 0.254) (layer "F.Cu") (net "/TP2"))
 (segment (start 162.5 98) (end 162.5 98.85) (width 0.254) (layer "F.Cu") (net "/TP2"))
 (segment (start 135.306626 97.7264) (end 135 98.033026) (width 0.254) (layer "F.Cu") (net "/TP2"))
 (segment (start 177.6936 92.923) (end 169.237 92.923) (width 0.254) (layer "F.Cu") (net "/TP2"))
 (segment (start 169.237 92.923) (end 168.16 94) (width 0.254) (layer "F.Cu") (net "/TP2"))
 (segment (start 183.749999 101.954993) (end 183.749999 99.749999) (width 0.254) (layer "F.Cu") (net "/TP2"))
 (segment (start 165.269 95.231) (end 162.5 98) (width 0.254) (layer "F.Cu") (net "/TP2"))
 (segment (start 177.923 93.1524) (end 177.6936 92.923) (width 0.254) (layer "F.Cu") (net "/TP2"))
 (segment (start 135 98.033026) (end 135 99.25) (width 0.254) (layer "F.Cu") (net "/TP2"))
 (segment (start 179.5 94.5) (end 183.749999 98.749999) (width 0.254) (layer "F.Cu") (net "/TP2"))
 (via (at 179.5 94.5) (size 0.7128) (drill 0.3048) (layers "F.Cu" "B.Cu") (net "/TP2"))
 (via (at 136 97.7264) (size 0.7128) (drill 0.3048) (layers "F.Cu" "B.Cu") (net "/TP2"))
 (via (at 180.5 96.5) (size 0.7128) (drill 0.3048) (layers "F.Cu" "B.Cu") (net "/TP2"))
 (via (at 177.923 93.1524) (size 0.7128) (drill 0.3048) (layers "F.Cu" "B.Cu") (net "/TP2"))
 (segment (start 180.981 96.019) (end 180.981 94.300763) (width 0.254) (layer "B.Cu") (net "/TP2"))
 (segment (start 180.981 94.300763) (end 178.895237 92.215) (width 0.254) (layer "B.Cu") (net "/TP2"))
 (segment (start 178.1524 93.1524) (end 177.923 93.1524) (width 0.254) (layer "B.Cu") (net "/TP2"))
 (segment (start 161.000842 97.515998) (end 161.00884 97.508) (width 0.254) (layer "B.Cu") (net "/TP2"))
 (segment (start 159.171263 97.523997) (end 159.17926 97.516) (width 0.254) (layer "B.Cu") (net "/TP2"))
 (segment (start 180.5 96.5) (end 180.981 96.019) (width 0.254) (layer "B.Cu") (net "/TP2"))
 (segment (start 178.895237 92.215) (end 169.945 92.215) (width 0.254) (layer "B.Cu") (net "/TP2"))
 (segment (start 136 97.7264) (end 136.075402 97.650998) (width 0.254) (layer "B.Cu") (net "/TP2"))
 (segment (start 136.683868 97.650998) (end 136.810866 97.524) (width 0.254) (layer "B.Cu") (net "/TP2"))
 (segment (start 161.00884 97.508) (end 162.830421 97.507999) (width 0.254) (layer "B.Cu") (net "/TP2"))
 (segment (start 179.5 94.5) (end 178.1524 93.1524) (width 0.254) (layer "B.Cu") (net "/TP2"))
 (segment (start 164.66 97.5) (end 168.16 94) (width 0.254) (layer "B.Cu") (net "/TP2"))
 (segment (start 162.83842 97.5) (end 164.66 97.5) (width 0.254) (layer "B.Cu") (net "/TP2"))
 (segment (start 169.945 92.215) (end 168.16 94) (width 0.254) (layer "B.Cu") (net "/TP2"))
 (segment (start 136.075402 97.650998) (end 136.683868 97.650998) (width 0.254) (layer "B.Cu") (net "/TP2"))
 (segment (start 162.830421 97.507999) (end 162.83842 97.5) (width 0.254) (layer "B.Cu") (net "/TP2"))
 (segment (start 136.810866 97.524) (end 159.171263 97.523997) (width 0.254) (layer "B.Cu") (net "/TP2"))
 (segment (start 159.17926 97.516) (end 161.000842 97.515998) (width 0.254) (layer "B.Cu") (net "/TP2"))
 (segment (start 163.5 97.783) (end 163.5 98.85) (width 0.254) (layer "F.Cu") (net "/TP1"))
 (segment (start 180 94) (end 184.250001 98.250001) (width 0.254) (layer "F.Cu") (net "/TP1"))
 (segment (start 136.429 98.159) (end 138.5 98.159) (width 0.254) (layer "F.Cu") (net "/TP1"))
 (segment (start 136 99.25) (end 136 98.588) (width 0.254) (layer "F.Cu") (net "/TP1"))
 (segment (start 179.427592 93.5834) (end 179.844192 94) (width 0.254) (layer "F.Cu") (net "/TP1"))
 (segment (start 179.844192 94) (end 180 94) (width 0.254) (layer "F.Cu") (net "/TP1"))
 (segment (start 165.283 96) (end 163.5 97.783) (width 0.254) (layer "F.Cu") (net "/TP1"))
 (segment (start 184.250001 98.250001) (end 184.250001 101.954993) (width 0.254) (layer "F.Cu") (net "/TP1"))
 (segment (start 136 98.588) (end 136.429 98.159) (width 0.254) (layer "F.Cu") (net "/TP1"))
 (segment (start 168.7 96) (end 165.283 96) (width 0.254) (layer "F.Cu") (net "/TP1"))
 (segment (start 170.7 94) (end 168.7 96) (width 0.254) (layer "F.Cu") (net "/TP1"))
 (via (at 138.5 98.159) (size 0.7128) (drill 0.3048) (layers "F.Cu" "B.Cu") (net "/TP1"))
 (via (at 179.427592 93.5834) (size 0.7128) (drill 0.3048) (layers "F.Cu" "B.Cu") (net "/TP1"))
 (segment (start 172.131 92.569) (end 170.7 94) (width 0.254) (layer "B.Cu") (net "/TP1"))
 (segment (start 138.5 98.159) (end 166.541 98.159) (width 0.254) (layer "B.Cu") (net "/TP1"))
 (segment (start 179.427592 93.427592) (end 178.569 92.569) (width 0.254) (layer "B.Cu") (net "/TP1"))
 (segment (start 178.569 92.569) (end 172.131 92.569) (width 0.254) (layer "B.Cu") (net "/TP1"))
 (segment (start 179.427592 93.5834) (end 179.427592 93.427592) (width 0.254) (layer "B.Cu") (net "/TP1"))
 (segment (start 166.541 98.159) (end 170.7 94) (width 0.254) (layer "B.Cu") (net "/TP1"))
 (segment (start 165.25071 96.75071) (end 164.5 97.50142) (width 0.254) (layer "F.Cu") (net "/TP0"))
 (segment (start 178 94) (end 173.24 94) (width 0.254) (layer "F.Cu") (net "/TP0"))
 (segment (start 137 99.25) (end 141.25 99.25) (width 0.254) (layer "F.Cu") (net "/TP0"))
 (segment (start 180 93) (end 179 93) (width 0.254) (layer "F.Cu") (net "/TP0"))
 (segment (start 170.48929 96.75071) (end 165.25071 96.75071) (width 0.254) (layer "F.Cu") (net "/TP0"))
 (segment (start 173.24 94) (end 170.48929 96.75071) (width 0.254) (layer "F.Cu") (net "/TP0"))
 (segment (start 184.75 101.954993) (end 184.75 97.75) (width 0.254) (layer "F.Cu") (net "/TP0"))
 (segment (start 164.5 97.50142) (end 164.5 98.85) (width 0.254) (layer "F.Cu") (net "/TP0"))
 (segment (start 179 93) (end 178 94) (width 0.254) (layer "F.Cu") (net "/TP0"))
 (segment (start 184.75 97.75) (end 180 93) (width 0.254) (layer "F.Cu") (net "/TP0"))
 (segment (start 141.25 99.25) (end 141.5 99) (width 0.254) (layer "F.Cu") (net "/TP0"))
 (via (at 141.5 99) (size 0.7128) (drill 0.3048) (layers "F.Cu" "B.Cu") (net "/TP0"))
 (segment (start 141.5 99) (end 168.24 99) (width 0.254) (layer "B.Cu") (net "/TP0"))
 (segment (start 168.24 99) (end 173.24 94) (width 0.254) (layer "B.Cu") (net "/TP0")))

